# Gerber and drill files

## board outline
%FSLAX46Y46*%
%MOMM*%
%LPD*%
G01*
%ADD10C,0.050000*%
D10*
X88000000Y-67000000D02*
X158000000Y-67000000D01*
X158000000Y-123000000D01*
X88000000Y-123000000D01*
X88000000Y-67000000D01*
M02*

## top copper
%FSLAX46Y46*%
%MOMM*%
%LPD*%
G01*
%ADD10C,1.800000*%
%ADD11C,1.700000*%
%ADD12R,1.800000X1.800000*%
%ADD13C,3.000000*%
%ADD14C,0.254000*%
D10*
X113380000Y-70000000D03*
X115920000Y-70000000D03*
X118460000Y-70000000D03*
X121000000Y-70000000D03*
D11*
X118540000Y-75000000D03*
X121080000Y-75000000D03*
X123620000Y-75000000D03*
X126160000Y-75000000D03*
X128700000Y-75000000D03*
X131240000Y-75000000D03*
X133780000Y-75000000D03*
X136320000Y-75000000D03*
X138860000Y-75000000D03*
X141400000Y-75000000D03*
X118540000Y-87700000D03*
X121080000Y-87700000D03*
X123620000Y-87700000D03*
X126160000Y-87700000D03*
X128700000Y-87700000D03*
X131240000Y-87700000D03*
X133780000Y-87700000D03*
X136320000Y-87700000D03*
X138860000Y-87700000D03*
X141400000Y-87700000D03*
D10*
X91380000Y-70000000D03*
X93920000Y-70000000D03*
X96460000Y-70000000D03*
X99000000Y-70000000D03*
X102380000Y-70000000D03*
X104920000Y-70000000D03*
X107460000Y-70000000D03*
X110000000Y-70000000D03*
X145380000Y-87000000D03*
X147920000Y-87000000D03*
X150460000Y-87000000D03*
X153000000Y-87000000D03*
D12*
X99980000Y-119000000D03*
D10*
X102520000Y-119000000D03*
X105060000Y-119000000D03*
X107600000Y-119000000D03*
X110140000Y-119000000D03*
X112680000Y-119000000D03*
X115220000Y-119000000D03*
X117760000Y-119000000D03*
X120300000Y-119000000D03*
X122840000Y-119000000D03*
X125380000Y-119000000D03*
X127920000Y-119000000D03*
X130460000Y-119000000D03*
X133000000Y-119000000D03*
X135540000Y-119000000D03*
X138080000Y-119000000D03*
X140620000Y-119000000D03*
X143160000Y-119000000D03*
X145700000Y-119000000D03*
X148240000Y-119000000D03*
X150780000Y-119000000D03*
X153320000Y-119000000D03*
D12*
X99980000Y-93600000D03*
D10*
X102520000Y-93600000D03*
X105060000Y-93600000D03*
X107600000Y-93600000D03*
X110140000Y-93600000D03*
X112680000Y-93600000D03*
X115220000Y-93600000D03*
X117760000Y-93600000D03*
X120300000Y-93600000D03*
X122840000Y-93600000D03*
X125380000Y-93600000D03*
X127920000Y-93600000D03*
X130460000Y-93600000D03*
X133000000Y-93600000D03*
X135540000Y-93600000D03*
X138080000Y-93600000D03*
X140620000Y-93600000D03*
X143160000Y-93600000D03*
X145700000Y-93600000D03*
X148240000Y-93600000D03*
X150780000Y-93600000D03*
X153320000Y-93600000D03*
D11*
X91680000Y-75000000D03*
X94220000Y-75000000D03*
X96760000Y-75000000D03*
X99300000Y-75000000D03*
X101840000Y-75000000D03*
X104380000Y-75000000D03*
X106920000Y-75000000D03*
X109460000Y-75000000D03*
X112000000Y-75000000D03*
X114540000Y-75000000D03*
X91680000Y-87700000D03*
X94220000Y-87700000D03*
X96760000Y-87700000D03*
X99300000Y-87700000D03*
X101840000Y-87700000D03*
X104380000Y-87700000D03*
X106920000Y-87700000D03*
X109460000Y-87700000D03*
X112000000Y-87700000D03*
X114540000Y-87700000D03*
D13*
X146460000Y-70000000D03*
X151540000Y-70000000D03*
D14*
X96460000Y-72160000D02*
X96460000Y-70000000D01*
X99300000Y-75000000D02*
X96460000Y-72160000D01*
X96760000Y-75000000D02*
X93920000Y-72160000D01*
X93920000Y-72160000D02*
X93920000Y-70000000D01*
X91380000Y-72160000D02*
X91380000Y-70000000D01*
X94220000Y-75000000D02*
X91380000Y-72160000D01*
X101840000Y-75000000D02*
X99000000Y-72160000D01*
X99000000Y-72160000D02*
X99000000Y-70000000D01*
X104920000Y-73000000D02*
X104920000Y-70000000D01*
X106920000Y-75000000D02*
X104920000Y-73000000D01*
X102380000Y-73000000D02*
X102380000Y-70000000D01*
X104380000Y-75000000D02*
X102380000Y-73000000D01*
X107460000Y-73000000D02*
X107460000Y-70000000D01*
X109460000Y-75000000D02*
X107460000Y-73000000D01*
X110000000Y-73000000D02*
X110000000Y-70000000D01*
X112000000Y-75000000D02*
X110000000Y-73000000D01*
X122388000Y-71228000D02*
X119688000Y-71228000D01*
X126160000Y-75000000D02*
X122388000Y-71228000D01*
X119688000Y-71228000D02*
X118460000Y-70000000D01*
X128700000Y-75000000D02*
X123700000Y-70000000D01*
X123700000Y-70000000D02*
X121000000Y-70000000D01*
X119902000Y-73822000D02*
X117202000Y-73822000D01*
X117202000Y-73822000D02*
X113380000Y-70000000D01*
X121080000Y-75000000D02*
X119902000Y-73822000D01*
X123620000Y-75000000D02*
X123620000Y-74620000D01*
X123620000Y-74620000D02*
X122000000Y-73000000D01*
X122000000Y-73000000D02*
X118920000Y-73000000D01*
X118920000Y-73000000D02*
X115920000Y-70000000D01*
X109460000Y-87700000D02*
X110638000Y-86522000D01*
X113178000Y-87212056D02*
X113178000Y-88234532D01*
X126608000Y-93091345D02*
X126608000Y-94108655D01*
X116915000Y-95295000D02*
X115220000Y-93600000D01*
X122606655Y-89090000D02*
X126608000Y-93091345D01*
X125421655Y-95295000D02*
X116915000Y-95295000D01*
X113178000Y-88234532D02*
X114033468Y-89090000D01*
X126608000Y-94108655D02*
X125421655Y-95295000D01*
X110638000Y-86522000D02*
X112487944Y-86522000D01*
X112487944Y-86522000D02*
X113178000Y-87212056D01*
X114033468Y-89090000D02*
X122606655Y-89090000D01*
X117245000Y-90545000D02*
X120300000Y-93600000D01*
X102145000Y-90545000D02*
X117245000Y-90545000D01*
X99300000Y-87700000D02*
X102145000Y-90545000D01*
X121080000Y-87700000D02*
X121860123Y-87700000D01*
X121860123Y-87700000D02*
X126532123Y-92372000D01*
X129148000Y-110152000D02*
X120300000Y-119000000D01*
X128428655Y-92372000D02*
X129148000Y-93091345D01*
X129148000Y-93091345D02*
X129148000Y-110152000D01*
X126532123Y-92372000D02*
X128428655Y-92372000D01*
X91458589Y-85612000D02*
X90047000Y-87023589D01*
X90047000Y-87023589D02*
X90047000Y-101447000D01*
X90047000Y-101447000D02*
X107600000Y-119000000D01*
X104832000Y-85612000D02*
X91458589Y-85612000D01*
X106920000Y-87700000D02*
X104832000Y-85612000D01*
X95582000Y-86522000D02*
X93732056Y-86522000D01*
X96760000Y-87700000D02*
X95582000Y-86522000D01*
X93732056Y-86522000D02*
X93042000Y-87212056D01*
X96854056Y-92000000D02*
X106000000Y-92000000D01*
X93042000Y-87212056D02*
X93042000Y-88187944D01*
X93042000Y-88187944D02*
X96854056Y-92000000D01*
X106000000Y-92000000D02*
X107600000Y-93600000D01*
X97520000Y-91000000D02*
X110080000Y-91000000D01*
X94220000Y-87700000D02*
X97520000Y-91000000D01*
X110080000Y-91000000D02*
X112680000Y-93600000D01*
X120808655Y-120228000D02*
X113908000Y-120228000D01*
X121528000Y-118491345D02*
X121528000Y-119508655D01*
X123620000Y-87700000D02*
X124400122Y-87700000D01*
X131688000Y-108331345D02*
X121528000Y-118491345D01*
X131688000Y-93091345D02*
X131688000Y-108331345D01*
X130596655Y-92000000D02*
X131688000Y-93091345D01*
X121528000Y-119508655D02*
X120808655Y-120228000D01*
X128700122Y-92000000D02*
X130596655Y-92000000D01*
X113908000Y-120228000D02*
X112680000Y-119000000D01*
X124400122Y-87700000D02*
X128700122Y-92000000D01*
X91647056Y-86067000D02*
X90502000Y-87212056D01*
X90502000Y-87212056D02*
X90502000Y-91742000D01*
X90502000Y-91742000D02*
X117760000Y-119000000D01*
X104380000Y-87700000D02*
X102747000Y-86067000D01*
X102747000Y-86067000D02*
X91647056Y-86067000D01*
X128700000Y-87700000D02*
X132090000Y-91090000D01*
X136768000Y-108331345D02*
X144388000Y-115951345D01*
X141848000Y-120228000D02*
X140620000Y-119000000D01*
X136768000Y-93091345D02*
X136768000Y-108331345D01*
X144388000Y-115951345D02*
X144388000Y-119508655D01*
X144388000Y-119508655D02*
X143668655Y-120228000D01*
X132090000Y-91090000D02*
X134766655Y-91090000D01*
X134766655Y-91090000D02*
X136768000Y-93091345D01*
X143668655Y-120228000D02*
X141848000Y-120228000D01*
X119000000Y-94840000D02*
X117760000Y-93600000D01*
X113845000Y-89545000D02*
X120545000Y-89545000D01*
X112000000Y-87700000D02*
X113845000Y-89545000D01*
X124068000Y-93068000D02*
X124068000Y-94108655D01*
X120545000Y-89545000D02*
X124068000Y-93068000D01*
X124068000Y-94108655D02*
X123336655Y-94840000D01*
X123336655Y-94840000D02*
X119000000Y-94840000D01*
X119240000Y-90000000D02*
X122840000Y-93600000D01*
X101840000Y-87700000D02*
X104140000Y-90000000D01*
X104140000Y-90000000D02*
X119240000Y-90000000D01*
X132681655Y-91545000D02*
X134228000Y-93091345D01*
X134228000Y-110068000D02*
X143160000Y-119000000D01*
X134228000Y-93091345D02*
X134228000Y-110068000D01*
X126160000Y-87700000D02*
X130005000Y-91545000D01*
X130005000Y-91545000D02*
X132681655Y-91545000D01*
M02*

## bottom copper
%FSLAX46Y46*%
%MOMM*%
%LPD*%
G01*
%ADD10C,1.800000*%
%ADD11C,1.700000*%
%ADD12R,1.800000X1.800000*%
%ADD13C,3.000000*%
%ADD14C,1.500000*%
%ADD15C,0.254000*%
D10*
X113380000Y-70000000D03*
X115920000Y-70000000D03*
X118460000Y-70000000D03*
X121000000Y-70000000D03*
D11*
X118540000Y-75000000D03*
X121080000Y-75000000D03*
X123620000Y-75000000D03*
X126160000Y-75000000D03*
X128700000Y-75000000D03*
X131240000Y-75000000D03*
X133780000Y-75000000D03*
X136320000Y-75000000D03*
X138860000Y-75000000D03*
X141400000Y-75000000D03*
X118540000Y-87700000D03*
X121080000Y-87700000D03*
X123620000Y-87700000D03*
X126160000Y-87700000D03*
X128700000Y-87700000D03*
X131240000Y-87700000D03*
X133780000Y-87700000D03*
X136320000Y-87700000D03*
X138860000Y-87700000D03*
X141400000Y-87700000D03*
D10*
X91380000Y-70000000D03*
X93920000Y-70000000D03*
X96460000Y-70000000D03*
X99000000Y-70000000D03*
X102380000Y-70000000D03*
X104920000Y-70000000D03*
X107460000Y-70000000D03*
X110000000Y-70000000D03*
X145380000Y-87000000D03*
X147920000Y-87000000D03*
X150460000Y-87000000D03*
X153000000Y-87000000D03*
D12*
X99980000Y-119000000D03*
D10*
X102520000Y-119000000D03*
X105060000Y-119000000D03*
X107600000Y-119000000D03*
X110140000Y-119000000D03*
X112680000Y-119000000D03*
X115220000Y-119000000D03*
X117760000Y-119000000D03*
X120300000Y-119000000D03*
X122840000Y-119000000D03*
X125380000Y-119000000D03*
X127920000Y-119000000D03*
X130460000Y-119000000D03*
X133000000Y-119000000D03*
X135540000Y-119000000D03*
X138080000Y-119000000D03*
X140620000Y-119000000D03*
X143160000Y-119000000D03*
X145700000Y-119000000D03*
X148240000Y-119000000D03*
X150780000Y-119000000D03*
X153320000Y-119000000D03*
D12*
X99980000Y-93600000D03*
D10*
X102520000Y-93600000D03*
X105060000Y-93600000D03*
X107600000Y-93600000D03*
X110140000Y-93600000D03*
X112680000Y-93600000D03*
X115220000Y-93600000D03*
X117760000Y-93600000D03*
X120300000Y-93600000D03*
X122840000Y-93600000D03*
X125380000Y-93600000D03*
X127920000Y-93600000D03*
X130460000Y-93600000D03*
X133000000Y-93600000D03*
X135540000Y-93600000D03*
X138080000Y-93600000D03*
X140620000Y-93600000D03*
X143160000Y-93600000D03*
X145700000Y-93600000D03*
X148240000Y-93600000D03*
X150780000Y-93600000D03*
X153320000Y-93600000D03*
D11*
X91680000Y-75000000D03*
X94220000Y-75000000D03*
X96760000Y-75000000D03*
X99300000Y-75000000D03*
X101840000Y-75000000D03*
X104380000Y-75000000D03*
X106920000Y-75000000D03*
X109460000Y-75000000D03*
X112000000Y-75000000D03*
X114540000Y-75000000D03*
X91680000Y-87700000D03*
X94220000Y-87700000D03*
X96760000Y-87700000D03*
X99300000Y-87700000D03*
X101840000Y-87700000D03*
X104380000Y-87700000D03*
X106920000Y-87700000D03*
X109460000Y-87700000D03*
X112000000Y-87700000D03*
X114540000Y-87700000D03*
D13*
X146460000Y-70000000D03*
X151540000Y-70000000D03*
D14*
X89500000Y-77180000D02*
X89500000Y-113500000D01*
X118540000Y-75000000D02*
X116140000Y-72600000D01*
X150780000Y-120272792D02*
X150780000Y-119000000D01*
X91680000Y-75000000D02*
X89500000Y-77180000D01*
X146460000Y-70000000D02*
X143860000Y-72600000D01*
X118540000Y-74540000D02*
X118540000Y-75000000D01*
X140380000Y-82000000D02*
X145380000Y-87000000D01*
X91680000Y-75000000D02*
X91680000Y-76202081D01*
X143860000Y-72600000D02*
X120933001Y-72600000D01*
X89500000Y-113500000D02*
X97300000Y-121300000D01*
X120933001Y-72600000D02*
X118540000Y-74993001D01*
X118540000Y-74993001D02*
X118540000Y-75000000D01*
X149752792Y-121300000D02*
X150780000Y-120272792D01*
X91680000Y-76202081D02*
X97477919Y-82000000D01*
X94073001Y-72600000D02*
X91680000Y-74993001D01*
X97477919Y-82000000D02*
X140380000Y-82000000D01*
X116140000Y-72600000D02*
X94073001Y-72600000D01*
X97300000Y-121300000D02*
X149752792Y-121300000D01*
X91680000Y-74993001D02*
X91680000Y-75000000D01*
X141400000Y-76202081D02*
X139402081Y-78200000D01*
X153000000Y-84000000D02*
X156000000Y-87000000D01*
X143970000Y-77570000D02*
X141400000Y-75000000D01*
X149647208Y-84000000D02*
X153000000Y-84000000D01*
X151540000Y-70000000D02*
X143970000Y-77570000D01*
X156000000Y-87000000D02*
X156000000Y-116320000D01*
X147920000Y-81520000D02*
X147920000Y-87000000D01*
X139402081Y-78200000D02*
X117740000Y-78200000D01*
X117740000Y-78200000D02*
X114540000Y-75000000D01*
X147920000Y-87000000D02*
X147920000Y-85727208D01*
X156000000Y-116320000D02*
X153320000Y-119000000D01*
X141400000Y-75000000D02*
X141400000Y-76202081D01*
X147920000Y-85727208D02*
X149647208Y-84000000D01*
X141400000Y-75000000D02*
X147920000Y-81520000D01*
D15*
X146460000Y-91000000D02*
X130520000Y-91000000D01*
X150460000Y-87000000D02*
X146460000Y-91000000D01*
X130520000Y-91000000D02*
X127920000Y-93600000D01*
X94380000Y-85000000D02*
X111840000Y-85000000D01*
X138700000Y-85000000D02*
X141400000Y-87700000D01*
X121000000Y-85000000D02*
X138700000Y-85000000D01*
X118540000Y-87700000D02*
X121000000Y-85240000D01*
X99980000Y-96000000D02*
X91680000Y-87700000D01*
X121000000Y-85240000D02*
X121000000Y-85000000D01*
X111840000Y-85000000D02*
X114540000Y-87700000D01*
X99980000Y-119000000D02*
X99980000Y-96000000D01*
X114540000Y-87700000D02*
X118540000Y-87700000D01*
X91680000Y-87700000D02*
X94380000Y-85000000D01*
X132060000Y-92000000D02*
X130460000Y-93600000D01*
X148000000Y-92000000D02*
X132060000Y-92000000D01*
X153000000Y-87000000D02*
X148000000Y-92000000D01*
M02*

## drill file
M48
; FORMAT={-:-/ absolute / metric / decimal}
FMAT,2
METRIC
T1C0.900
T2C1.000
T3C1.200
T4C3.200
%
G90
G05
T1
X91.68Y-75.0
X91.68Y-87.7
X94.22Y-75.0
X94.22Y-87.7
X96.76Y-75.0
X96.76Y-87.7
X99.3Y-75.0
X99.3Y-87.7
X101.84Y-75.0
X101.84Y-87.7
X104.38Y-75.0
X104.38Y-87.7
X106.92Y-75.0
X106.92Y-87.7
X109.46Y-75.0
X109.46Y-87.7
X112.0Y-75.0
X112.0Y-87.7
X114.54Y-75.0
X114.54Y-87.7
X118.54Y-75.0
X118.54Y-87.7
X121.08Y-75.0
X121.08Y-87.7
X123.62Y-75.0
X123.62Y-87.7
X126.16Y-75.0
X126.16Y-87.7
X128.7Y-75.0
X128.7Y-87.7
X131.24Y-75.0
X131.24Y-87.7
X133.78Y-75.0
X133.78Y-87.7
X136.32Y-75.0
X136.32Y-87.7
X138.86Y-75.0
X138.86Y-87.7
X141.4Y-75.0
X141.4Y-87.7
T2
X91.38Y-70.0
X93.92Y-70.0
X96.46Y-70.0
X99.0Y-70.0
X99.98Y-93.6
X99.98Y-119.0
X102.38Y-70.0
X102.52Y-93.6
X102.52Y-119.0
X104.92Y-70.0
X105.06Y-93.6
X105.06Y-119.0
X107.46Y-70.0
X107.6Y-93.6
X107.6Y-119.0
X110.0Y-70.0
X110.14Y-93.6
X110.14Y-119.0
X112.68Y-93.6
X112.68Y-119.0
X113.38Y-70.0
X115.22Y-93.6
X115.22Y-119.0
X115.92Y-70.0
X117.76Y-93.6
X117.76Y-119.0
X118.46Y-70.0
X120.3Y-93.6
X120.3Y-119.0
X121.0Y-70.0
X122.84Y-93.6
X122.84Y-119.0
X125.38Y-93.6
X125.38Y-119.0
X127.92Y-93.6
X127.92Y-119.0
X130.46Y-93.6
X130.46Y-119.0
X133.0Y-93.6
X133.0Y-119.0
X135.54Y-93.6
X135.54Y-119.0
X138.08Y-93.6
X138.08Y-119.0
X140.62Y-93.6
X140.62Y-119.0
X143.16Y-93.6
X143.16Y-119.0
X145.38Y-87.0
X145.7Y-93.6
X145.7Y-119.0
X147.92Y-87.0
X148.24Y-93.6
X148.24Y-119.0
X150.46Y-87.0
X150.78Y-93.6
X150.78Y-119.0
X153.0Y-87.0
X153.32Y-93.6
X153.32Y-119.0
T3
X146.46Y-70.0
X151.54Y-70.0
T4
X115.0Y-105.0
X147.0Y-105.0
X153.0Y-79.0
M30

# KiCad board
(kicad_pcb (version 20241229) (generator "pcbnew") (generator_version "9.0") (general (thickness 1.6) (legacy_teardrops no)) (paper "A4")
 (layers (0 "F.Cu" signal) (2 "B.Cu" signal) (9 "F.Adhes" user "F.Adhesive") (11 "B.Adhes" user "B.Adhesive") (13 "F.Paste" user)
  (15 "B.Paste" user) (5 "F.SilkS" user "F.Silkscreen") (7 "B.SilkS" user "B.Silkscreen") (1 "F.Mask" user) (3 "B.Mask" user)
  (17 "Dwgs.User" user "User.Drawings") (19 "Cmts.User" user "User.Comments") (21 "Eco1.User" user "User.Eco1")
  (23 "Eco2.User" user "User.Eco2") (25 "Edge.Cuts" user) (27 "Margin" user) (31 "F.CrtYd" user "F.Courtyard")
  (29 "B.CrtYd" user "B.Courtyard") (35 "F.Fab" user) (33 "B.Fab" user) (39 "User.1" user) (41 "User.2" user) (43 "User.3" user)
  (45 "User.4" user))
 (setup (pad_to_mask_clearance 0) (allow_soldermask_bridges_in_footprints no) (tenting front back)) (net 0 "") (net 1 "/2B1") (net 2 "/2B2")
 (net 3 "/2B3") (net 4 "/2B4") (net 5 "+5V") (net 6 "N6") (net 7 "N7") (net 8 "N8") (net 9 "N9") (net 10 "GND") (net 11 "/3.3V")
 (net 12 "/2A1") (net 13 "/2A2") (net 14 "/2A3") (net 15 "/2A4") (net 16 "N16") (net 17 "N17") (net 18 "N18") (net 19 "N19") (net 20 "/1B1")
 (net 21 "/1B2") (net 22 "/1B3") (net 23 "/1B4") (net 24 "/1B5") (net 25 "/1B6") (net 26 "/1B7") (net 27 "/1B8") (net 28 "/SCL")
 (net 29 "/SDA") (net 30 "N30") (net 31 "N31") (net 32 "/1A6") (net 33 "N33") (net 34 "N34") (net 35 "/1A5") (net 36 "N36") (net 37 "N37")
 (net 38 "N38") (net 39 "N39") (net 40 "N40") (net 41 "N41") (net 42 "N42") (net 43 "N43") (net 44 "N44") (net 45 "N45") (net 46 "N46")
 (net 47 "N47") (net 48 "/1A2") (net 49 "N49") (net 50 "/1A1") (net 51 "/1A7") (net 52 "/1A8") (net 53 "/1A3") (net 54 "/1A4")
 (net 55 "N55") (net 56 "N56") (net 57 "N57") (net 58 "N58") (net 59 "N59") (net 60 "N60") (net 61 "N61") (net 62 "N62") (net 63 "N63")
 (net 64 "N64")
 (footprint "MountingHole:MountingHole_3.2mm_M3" (layer "F.Cu") (at 153 79)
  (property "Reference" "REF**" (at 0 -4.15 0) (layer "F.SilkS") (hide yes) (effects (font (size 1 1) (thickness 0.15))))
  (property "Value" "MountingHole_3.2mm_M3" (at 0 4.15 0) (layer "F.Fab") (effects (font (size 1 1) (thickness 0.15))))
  (pad "" np_thru_hole circle (at 0 0) (size 3.2 3.2) (drill 3.2) (layers "*.Cu" "*.Mask")))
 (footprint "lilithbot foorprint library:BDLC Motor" (layer "F.Cu") (at 117.19 70.254)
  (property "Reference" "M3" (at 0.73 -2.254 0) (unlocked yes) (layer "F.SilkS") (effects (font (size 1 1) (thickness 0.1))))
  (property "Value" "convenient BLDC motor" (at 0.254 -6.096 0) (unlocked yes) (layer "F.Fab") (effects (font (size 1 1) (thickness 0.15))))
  (pad "1" thru_hole circle (at -3.81 -0.254) (size 1.8 1.8) (drill 1) (layers "*.Cu" "*.Mask") (remove_unused_layers no) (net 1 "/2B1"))
  (pad "2" thru_hole circle (at -1.27 -0.254) (size 1.8 1.8) (drill 1) (layers "*.Cu" "*.Mask") (remove_unused_layers no) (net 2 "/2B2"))
  (pad "3" thru_hole circle (at 1.27 -0.254) (size 1.8 1.8) (drill 1) (layers "*.Cu" "*.Mask") (remove_unused_layers no) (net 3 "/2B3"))
  (pad "4" thru_hole circle (at 3.81 -0.254) (size 1.8 1.8) (drill 1) (layers "*.Cu" "*.Mask") (remove_unused_layers no) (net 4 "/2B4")))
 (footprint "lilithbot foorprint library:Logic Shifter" (layer "F.Cu") (at 130.944878 82.58)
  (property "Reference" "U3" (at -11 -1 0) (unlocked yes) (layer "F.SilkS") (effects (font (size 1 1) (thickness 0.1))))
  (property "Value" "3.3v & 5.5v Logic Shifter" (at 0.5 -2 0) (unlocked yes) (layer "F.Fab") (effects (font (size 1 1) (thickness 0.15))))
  (pad "1" thru_hole circle (at -12.404878 -7.58) (size 1.7 1.7) (drill 0.9) (layers "*.Cu" "*.Mask") (remove_unused_layers no)
   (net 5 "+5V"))
  (pad "2" thru_hole circle (at -9.864878 -7.58) (size 1.7 1.7) (drill 0.9) (layers "*.Cu" "*.Mask") (remove_unused_layers no)
   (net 1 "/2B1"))
  (pad "3" thru_hole circle (at -7.324878 -7.58) (size 1.7 1.7) (drill 0.9) (layers "*.Cu" "*.Mask") (remove_unused_layers no)
   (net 2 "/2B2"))
  (pad "4" thru_hole circle (at -4.784878 -7.58) (size 1.7 1.7) (drill 0.9) (layers "*.Cu" "*.Mask") (remove_unused_layers no)
   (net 3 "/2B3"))
  (pad "5" thru_hole circle (at -2.244878 -7.58) (size 1.7 1.7) (drill 0.9) (layers "*.Cu" "*.Mask") (remove_unused_layers no)
   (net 4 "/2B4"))
  (pad "6" thru_hole circle (at 0.295122 -7.58) (size 1.7 1.7) (drill 0.9) (layers "*.Cu" "*.Mask") (remove_unused_layers no) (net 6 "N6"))
  (pad "7" thru_hole circle (at 2.835122 -7.58) (size 1.7 1.7) (drill 0.9) (layers "*.Cu" "*.Mask") (remove_unused_layers no) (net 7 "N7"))
  (pad "8" thru_hole circle (at 5.375122 -7.58) (size 1.7 1.7) (drill 0.9) (layers "*.Cu" "*.Mask") (remove_unused_layers no) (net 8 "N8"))
  (pad "9" thru_hole circle (at 7.915122 -7.58) (size 1.7 1.7) (drill 0.9) (layers "*.Cu" "*.Mask") (remove_unused_layers no) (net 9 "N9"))
  (pad "10" thru_hole circle (at 10.455122 -7.58) (size 1.7 1.7) (drill 0.9) (layers "*.Cu" "*.Mask") (remove_unused_layers no)
   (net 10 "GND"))
  (pad "11" thru_hole circle (at -12.404878 5.12) (size 1.7 1.7) (drill 0.9) (layers "*.Cu" "*.Mask") (remove_unused_layers no)
   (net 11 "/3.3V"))
  (pad "12" thru_hole circle (at -9.864878 5.12) (size 1.7 1.7) (drill 0.9) (layers "*.Cu" "*.Mask") (remove_unused_layers no)
   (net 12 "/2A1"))
  (pad "13" thru_hole circle (at -7.324878 5.12) (size 1.7 1.7) (drill 0.9) (layers "*.Cu" "*.Mask") (remove_unused_layers no)
   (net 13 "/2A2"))
  (pad "14" thru_hole circle (at -4.784878 5.12) (size 1.7 1.7) (drill 0.9) (layers "*.Cu" "*.Mask") (remove_unused_layers no)
   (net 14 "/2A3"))
  (pad "15" thru_hole circle (at -2.244878 5.12) (size 1.7 1.7) (drill 0.9) (layers "*.Cu" "*.Mask") (remove_unused_layers no)
   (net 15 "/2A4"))
  (pad "16" thru_hole circle (at 0.295122 5.12) (size 1.7 1.7) (drill 0.9) (layers "*.Cu" "*.Mask") (remove_unused_layers no) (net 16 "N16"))
  (pad "17" thru_hole circle (at 2.835122 5.12) (size 1.7 1.7) (drill 0.9) (layers "*.Cu" "*.Mask") (remove_unused_layers no) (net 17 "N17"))
  (pad "18" thru_hole circle (at 5.375122 5.12) (size 1.7 1.7) (drill 0.9) (layers "*.Cu" "*.Mask") (remove_unused_layers no) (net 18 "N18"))
  (pad "19" thru_hole circle (at 7.915122 5.12) (size 1.7 1.7) (drill 0.9) (layers "*.Cu" "*.Mask") (remove_unused_layers no) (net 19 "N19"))
  (pad "20" thru_hole circle (at 10.455122 5.12) (size 1.7 1.7) (drill 0.9) (layers "*.Cu" "*.Mask") (remove_unused_layers no)
   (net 11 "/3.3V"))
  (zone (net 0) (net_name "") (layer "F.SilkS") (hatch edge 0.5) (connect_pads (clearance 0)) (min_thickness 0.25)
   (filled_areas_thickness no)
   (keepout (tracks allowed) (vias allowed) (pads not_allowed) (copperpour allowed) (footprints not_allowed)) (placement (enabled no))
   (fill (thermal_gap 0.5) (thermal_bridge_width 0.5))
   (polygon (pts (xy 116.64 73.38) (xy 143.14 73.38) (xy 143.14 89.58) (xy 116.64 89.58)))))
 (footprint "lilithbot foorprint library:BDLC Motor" (layer "F.Cu") (at 95.19 70.254)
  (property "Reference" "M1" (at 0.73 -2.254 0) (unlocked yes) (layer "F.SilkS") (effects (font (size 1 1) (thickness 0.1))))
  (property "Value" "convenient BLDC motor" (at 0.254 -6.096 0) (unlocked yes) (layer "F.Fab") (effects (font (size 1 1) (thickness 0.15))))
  (pad "1" thru_hole circle (at -3.81 -0.254) (size 1.8 1.8) (drill 1) (layers "*.Cu" "*.Mask") (remove_unused_layers no) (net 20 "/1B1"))
  (pad "2" thru_hole circle (at -1.27 -0.254) (size 1.8 1.8) (drill 1) (layers "*.Cu" "*.Mask") (remove_unused_layers no) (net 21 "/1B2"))
  (pad "3" thru_hole circle (at 1.27 -0.254) (size 1.8 1.8) (drill 1) (layers "*.Cu" "*.Mask") (remove_unused_layers no) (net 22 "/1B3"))
  (pad "4" thru_hole circle (at 3.81 -0.254) (size 1.8 1.8) (drill 1) (layers "*.Cu" "*.Mask") (remove_unused_layers no) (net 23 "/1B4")))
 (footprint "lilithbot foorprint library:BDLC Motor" (layer "F.Cu") (at 106.19 70.254)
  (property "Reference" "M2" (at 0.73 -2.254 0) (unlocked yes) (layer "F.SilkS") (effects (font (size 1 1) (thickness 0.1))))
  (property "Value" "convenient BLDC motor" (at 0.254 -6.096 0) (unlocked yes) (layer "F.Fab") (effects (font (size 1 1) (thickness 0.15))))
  (pad "1" thru_hole circle (at -3.81 -0.254) (size 1.8 1.8) (drill 1) (layers "*.Cu" "*.Mask") (remove_unused_layers no) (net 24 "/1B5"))
  (pad "2" thru_hole circle (at -1.27 -0.254) (size 1.8 1.8) (drill 1) (layers "*.Cu" "*.Mask") (remove_unused_layers no) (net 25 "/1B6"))
  (pad "3" thru_hole circle (at 1.27 -0.254) (size 1.8 1.8) (drill 1) (layers "*.Cu" "*.Mask") (remove_unused_layers no) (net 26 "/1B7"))
  (pad "4" thru_hole circle (at 3.81 -0.254) (size 1.8 1.8) (drill 1) (layers "*.Cu" "*.Mask") (remove_unused_layers no) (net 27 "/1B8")))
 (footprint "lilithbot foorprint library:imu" (layer "F.Cu") (at 149.19 87)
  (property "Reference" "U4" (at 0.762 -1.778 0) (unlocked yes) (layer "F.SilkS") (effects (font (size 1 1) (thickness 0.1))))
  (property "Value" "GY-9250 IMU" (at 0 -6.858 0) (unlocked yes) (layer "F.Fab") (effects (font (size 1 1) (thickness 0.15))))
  (pad "1" thru_hole circle (at -3.81 0) (size 1.8 1.8) (drill 1) (layers "*.Cu" "*.Mask") (remove_unused_layers no) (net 5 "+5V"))
  (pad "2" thru_hole circle (at -1.27 0) (size 1.8 1.8) (drill 1) (layers "*.Cu" "*.Mask") (remove_unused_layers no) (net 10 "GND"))
  (pad "3" thru_hole circle (at 1.27 0) (size 1.8 1.8) (drill 1) (layers "*.Cu" "*.Mask") (remove_unused_layers no) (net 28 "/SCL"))
  (pad "4" thru_hole circle (at 3.81 0) (size 1.8 1.8) (drill 1) (layers "*.Cu" "*.Mask") (remove_unused_layers no) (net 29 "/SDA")))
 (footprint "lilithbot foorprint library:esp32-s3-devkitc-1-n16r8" (layer "F.Cu") (at 125.38 106.3 90)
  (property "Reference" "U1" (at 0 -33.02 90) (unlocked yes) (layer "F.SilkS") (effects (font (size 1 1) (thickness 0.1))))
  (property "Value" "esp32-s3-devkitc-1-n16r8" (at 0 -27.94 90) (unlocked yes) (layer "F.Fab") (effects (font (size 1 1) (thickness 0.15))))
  (pad "1" thru_hole rect (at -12.7 -25.4 90) (size 1.8 1.8) (drill 1) (layers "*.Cu" "*.Mask") (remove_unused_layers no) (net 11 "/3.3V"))
  (pad "2" thru_hole circle (at -12.7 -22.86 90) (size 1.8 1.8) (drill 1) (layers "*.Cu" "*.Mask") (remove_unused_layers no) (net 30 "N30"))
  (pad "3" thru_hole circle (at -12.7 -20.32 90) (size 1.8 1.8) (drill 1) (layers "*.Cu" "*.Mask") (remove_unused_layers no) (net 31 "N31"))
  (pad "4" thru_hole circle (at -12.7 -17.78 90) (size 1.8 1.8) (drill 1) (layers "*.Cu" "*.Mask") (remove_unused_layers no) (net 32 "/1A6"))
  (pad "5" thru_hole circle (at -12.7 -15.24 90) (size 1.8 1.8) (drill 1) (layers "*.Cu" "*.Mask") (remove_unused_layers no) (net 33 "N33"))
  (pad "6" thru_hole circle (at -12.7 -12.7 90) (size 1.8 1.8) (drill 1) (layers "*.Cu" "*.Mask") (remove_unused_layers no) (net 13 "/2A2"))
  (pad "7" thru_hole circle (at -12.7 -10.16 90) (size 1.8 1.8) (drill 1) (layers "*.Cu" "*.Mask") (remove_unused_layers no) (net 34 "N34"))
  (pad "8" thru_hole circle (at -12.7 -7.62 90) (size 1.8 1.8) (drill 1) (layers "*.Cu" "*.Mask") (remove_unused_layers no) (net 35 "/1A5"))
  (pad "9" thru_hole circle (at -12.7 -5.08 90) (size 1.8 1.8) (drill 1) (layers "*.Cu" "*.Mask") (remove_unused_layers no) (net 12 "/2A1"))
  (pad "10" thru_hole circle (at -12.7 -2.54 90) (size 1.8 1.8) (drill 1) (layers "*.Cu" "*.Mask") (remove_unused_layers no) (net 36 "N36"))
  (pad "11" thru_hole circle (at -12.7 0 90) (size 1.8 1.8) (drill 1) (layers "*.Cu" "*.Mask") (remove_unused_layers no) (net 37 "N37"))
  (pad "12" thru_hole circle (at -12.7 2.54 90) (size 1.8 1.8) (drill 1) (layers "*.Cu" "*.Mask") (remove_unused_layers no) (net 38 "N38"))
  (pad "13" thru_hole circle (at -12.7 5.08 90) (size 1.8 1.8) (drill 1) (layers "*.Cu" "*.Mask") (remove_unused_layers no) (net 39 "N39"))
  (pad "14" thru_hole circle (at -12.7 7.62 90) (size 1.8 1.8) (drill 1) (layers "*.Cu" "*.Mask") (remove_unused_layers no) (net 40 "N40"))
  (pad "15" thru_hole circle (at -12.7 10.16 90) (size 1.8 1.8) (drill 1) (layers "*.Cu" "*.Mask") (remove_unused_layers no) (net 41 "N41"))
  (pad "16" thru_hole circle (at -12.7 12.7 90) (size 1.8 1.8) (drill 1) (layers "*.Cu" "*.Mask") (remove_unused_layers no) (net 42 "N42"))
  (pad "17" thru_hole circle (at -12.7 15.24 90) (size 1.8 1.8) (drill 1) (layers "*.Cu" "*.Mask") (remove_unused_layers no) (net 15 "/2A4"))
  (pad "18" thru_hole circle (at -12.7 17.78 90) (size 1.8 1.8) (drill 1) (layers "*.Cu" "*.Mask") (remove_unused_layers no) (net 14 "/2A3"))
  (pad "19" thru_hole circle (at -12.7 20.32 90) (size 1.8 1.8) (drill 1) (layers "*.Cu" "*.Mask") (remove_unused_layers no) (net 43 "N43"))
  (pad "20" thru_hole circle (at -12.7 22.86 90) (size 1.8 1.8) (drill 1) (layers "*.Cu" "*.Mask") (remove_unused_layers no) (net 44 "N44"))
  (pad "21" thru_hole circle (at -12.7 25.4 90) (size 1.8 1.8) (drill 1) (layers "*.Cu" "*.Mask") (remove_unused_layers no) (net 5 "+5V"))
  (pad "22" thru_hole circle (at -12.7 27.94 90) (size 1.8 1.8) (drill 1) (layers "*.Cu" "*.Mask") (remove_unused_layers no) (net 10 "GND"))
  (pad "23" thru_hole rect (at 12.7 -25.4 90) (size 1.8 1.8) (drill 1) (layers "*.Cu" "*.Mask") (remove_unused_layers no) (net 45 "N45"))
  (pad "24" thru_hole circle (at 12.7 -22.86 90) (size 1.8 1.8) (drill 1) (layers "*.Cu" "*.Mask") (remove_unused_layers no) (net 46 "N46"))
  (pad "25" thru_hole circle (at 12.7 -20.32 90) (size 1.8 1.8) (drill 1) (layers "*.Cu" "*.Mask") (remove_unused_layers no) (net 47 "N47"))
  (pad "26" thru_hole circle (at 12.7 -17.78 90) (size 1.8 1.8) (drill 1) (layers "*.Cu" "*.Mask") (remove_unused_layers no) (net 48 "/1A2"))
  (pad "27" thru_hole circle (at 12.7 -15.24 90) (size 1.8 1.8) (drill 1) (layers "*.Cu" "*.Mask") (remove_unused_layers no) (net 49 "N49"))
  (pad "28" thru_hole circle (at 12.7 -12.7 90) (size 1.8 1.8) (drill 1) (layers "*.Cu" "*.Mask") (remove_unused_layers no) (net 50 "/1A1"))
  (pad "29" thru_hole circle (at 12.7 -10.16 90) (size 1.8 1.8) (drill 1) (layers "*.Cu" "*.Mask") (remove_unused_layers no) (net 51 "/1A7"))
  (pad "30" thru_hole circle (at 12.7 -7.62 90) (size 1.8 1.8) (drill 1) (layers "*.Cu" "*.Mask") (remove_unused_layers no) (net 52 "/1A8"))
  (pad "31" thru_hole circle (at 12.7 -5.08 90) (size 1.8 1.8) (drill 1) (layers "*.Cu" "*.Mask") (remove_unused_layers no) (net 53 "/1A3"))
  (pad "32" thru_hole circle (at 12.7 -2.54 90) (size 1.8 1.8) (drill 1) (layers "*.Cu" "*.Mask") (remove_unused_layers no) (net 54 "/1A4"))
  (pad "33" thru_hole circle (at 12.7 0 90) (size 1.8 1.8) (drill 1) (layers "*.Cu" "*.Mask") (remove_unused_layers no) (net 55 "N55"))
  (pad "34" thru_hole circle (at 12.7 2.54 90) (size 1.8 1.8) (drill 1) (layers "*.Cu" "*.Mask") (remove_unused_layers no) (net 28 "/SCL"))
  (pad "35" thru_hole circle (at 12.7 5.08 90) (size 1.8 1.8) (drill 1) (layers "*.Cu" "*.Mask") (remove_unused_layers no) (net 29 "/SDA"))
  (pad "36" thru_hole circle (at 12.7 7.62 90) (size 1.8 1.8) (drill 1) (layers "*.Cu" "*.Mask") (remove_unused_layers no) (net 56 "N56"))
  (pad "37" thru_hole circle (at 12.7 10.16 90) (size 1.8 1.8) (drill 1) (layers "*.Cu" "*.Mask") (remove_unused_layers no) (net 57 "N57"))
  (pad "38" thru_hole circle (at 12.7 12.7 90) (size 1.8 1.8) (drill 1) (layers "*.Cu" "*.Mask") (remove_unused_layers no) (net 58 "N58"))
  (pad "39" thru_hole circle (at 12.7 15.24 90) (size 1.8 1.8) (drill 1) (layers "*.Cu" "*.Mask") (remove_unused_layers no) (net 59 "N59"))
  (pad "40" thru_hole circle (at 12.7 17.78 90) (size 1.8 1.8) (drill 1) (layers "*.Cu" "*.Mask") (remove_unused_layers no) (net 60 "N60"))
  (pad "41" thru_hole circle (at 12.7 20.32 90) (size 1.8 1.8) (drill 1) (layers "*.Cu" "*.Mask") (remove_unused_layers no) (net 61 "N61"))
  (pad "42" thru_hole circle (at 12.7 22.86 90) (size 1.8 1.8) (drill 1) (layers "*.Cu" "*.Mask") (remove_unused_layers no) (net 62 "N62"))
  (pad "43" thru_hole circle (at 12.7 25.4 90) (size 1.8 1.8) (drill 1) (layers "*.Cu" "*.Mask") (remove_unused_layers no) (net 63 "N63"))
  (pad "44" thru_hole circle (at 12.7 27.94 90) (size 1.8 1.8) (drill 1) (layers "*.Cu" "*.Mask") (remove_unused_layers no) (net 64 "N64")))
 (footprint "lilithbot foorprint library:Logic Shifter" (layer "F.Cu") (at 104.084878 82.58)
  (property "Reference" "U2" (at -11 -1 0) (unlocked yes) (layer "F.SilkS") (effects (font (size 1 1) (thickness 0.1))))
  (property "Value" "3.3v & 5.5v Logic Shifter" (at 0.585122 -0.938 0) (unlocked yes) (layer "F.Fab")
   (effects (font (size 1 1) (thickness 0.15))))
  (pad "1" thru_hole circle (at -12.404878 -7.58) (size 1.7 1.7) (drill 0.9) (layers "*.Cu" "*.Mask") (remove_unused_layers no)
   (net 5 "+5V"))
  (pad "2" thru_hole circle (at -9.864878 -7.58) (size 1.7 1.7) (drill 0.9) (layers "*.Cu" "*.Mask") (remove_unused_layers no)
   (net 20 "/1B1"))
  (pad "3" thru_hole circle (at -7.324878 -7.58) (size 1.7 1.7) (drill 0.9) (layers "*.Cu" "*.Mask") (remove_unused_layers no)
   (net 21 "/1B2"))
  (pad "4" thru_hole circle (at -4.784878 -7.58) (size 1.7 1.7) (drill 0.9) (layers "*.Cu" "*.Mask") (remove_unused_layers no)
   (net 22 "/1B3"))
  (pad "5" thru_hole circle (at -2.244878 -7.58) (size 1.7 1.7) (drill 0.9) (layers "*.Cu" "*.Mask") (remove_unused_layers no)
   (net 23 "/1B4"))
  (pad "6" thru_hole circle (at 0.295122 -7.58) (size 1.7 1.7) (drill 0.9) (layers "*.Cu" "*.Mask") (remove_unused_layers no)
   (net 24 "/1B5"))
  (pad "7" thru_hole circle (at 2.835122 -7.58) (size 1.7 1.7) (drill 0.9) (layers "*.Cu" "*.Mask") (remove_unused_layers no)
   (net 25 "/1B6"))
  (pad "8" thru_hole circle (at 5.375122 -7.58) (size 1.7 1.7) (drill 0.9) (layers "*.Cu" "*.Mask") (remove_unused_layers no)
   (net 26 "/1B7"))
  (pad "9" thru_hole circle (at 7.915122 -7.58) (size 1.7 1.7) (drill 0.9) (layers "*.Cu" "*.Mask") (remove_unused_layers no)
   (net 27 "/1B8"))
  (pad "10" thru_hole circle (at 10.455122 -7.58) (size 1.7 1.7) (drill 0.9) (layers "*.Cu" "*.Mask") (remove_unused_layers no)
   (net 10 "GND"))
  (pad "11" thru_hole circle (at -12.404878 5.12) (size 1.7 1.7) (drill 0.9) (layers "*.Cu" "*.Mask") (remove_unused_layers no)
   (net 11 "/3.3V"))
  (pad "12" thru_hole circle (at -9.864878 5.12) (size 1.7 1.7) (drill 0.9) (layers "*.Cu" "*.Mask") (remove_unused_layers no)
   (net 50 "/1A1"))
  (pad "13" thru_hole circle (at -7.324878 5.12) (size 1.7 1.7) (drill 0.9) (layers "*.Cu" "*.Mask") (remove_unused_layers no)
   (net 48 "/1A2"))
  (pad "14" thru_hole circle (at -4.784878 5.12) (size 1.7 1.7) (drill 0.9) (layers "*.Cu" "*.Mask") (remove_unused_layers no)
   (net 53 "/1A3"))
  (pad "15" thru_hole circle (at -2.244878 5.12) (size 1.7 1.7) (drill 0.9) (layers "*.Cu" "*.Mask") (remove_unused_layers no)
   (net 54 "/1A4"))
  (pad "16" thru_hole circle (at 0.295122 5.12) (size 1.7 1.7) (drill 0.9) (layers "*.Cu" "*.Mask") (remove_unused_layers no)
   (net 35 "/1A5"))
  (pad "17" thru_hole circle (at 2.835122 5.12) (size 1.7 1.7) (drill 0.9) (layers "*.Cu" "*.Mask") (remove_unused_layers no)
   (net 32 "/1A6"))
  (pad "18" thru_hole circle (at 5.375122 5.12) (size 1.7 1.7) (drill 0.9) (layers "*.Cu" "*.Mask") (remove_unused_layers no)
   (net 51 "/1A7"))
  (pad "19" thru_hole circle (at 7.915122 5.12) (size 1.7 1.7) (drill 0.9) (layers "*.Cu" "*.Mask") (remove_unused_layers no)
   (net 52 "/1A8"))
  (pad "20" thru_hole circle (at 10.455122 5.12) (size 1.7 1.7) (drill 0.9) (layers "*.Cu" "*.Mask") (remove_unused_layers no)
   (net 11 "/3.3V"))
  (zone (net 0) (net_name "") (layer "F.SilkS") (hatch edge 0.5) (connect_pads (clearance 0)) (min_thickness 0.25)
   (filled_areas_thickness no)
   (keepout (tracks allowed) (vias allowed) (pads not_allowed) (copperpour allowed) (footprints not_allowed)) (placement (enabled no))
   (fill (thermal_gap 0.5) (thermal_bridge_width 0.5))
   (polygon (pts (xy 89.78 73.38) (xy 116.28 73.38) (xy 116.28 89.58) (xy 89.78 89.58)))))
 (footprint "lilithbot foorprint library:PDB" (layer "F.Cu") (at 149 70)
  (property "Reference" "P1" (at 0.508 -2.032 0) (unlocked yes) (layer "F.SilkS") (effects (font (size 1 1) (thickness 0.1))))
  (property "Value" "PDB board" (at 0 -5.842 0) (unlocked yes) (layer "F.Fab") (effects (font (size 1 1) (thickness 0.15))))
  (pad "1" thru_hole circle (at -2.54 0) (size 3 3) (drill 1.2) (layers "*.Cu" "*.Mask") (remove_unused_layers no) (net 5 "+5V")
   (thermal_bridge_width 0.5) (thermal_bridge_angle 90) (thermal_gap 0.25))
  (pad "2" thru_hole circle (at 2.54 0) (size 3 3) (drill 1.2) (layers "*.Cu" "*.Mask") (remove_unused_layers no) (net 10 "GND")
   (thermal_bridge_width 0.5) (thermal_bridge_angle 90) (thermal_gap 0.25)))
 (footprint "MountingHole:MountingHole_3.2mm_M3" (layer "F.Cu") (at 147 105)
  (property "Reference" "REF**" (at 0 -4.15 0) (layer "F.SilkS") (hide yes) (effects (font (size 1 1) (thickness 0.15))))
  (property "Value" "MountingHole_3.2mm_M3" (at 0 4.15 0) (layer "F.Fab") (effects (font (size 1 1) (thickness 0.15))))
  (pad "" np_thru_hole circle (at 0 0) (size 3.2 3.2) (drill 3.2) (layers "*.Cu" "*.Mask")))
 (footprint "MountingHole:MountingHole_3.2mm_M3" (layer "F.Cu") (at 115 105)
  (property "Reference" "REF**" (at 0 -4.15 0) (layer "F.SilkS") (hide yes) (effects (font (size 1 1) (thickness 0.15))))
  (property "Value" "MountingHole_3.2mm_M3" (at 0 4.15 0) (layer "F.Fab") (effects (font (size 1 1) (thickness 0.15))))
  (pad "" np_thru_hole circle (at 0 0) (size 3.2 3.2) (drill 3.2) (layers "*.Cu" "*.Mask")))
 (gr_rect (start 88 67) (end 158 123) (stroke (width 0.05) (type solid)) (fill no) (layer "Edge.Cuts"))
 (segment (start 96.46 72.16) (end 96.46 70) (width 0.254) (layer "F.Cu") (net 22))
 (segment (start 99.3 75) (end 96.46 72.16) (width 0.254) (layer "F.Cu") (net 22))
 (segment (start 96.76 75) (end 93.92 72.16) (width 0.254) (layer "F.Cu") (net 21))
 (segment (start 93.92 72.16) (end 93.92 70) (width 0.254) (layer "F.Cu") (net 21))
 (segment (start 91.38 72.16) (end 91.38 70) (width 0.254) (layer "F.Cu") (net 20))
 (segment (start 94.22 75) (end 91.38 72.16) (width 0.254) (layer "F.Cu") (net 20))
 (segment (start 101.84 75) (end 99 72.16) (width 0.254) (layer "F.Cu") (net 23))
 (segment (start 99 72.16) (end 99 70) (width 0.254) (layer "F.Cu") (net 23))
 (segment (start 104.92 73) (end 104.92 70) (width 0.254) (layer "F.Cu") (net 25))
 (segment (start 106.92 75) (end 104.92 73) (width 0.254) (layer "F.Cu") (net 25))
 (segment (start 102.38 73) (end 102.38 70) (width 0.254) (layer "F.Cu") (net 24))
 (segment (start 104.38 75) (end 102.38 73) (width 0.254) (layer "F.Cu") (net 24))
 (segment (start 107.46 73) (end 107.46 70) (width 0.254) (layer "F.Cu") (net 26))
 (segment (start 109.46 75) (end 107.46 73) (width 0.254) (layer "F.Cu") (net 26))
 (segment (start 110 73) (end 110 70) (width 0.254) (layer "F.Cu") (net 27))
 (segment (start 112 75) (end 110 73) (width 0.254) (layer "F.Cu") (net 27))
 (segment (start 122.388 71.228) (end 119.688 71.228) (width 0.254) (layer "F.Cu") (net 3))
 (segment (start 126.16 75) (end 122.388 71.228) (width 0.254) (layer "F.Cu") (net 3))
 (segment (start 119.688 71.228) (end 118.46 70) (width 0.254) (layer "F.Cu") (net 3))
 (segment (start 128.7 75) (end 123.7 70) (width 0.254) (layer "F.Cu") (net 4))
 (segment (start 123.7 70) (end 121 70) (width 0.254) (layer "F.Cu") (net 4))
 (segment (start 119.902 73.822) (end 117.202 73.822) (width 0.254) (layer "F.Cu") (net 1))
 (segment (start 117.202 73.822) (end 113.38 70) (width 0.254) (layer "F.Cu") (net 1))
 (segment (start 121.08 75) (end 119.902 73.822) (width 0.254) (layer "F.Cu") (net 1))
 (segment (start 123.62 75) (end 123.62 74.62) (width 0.254) (layer "F.Cu") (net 2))
 (segment (start 123.62 74.62) (end 122 73) (width 0.254) (layer "F.Cu") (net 2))
 (segment (start 122 73) (end 118.92 73) (width 0.254) (layer "F.Cu") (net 2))
 (segment (start 118.92 73) (end 115.92 70) (width 0.254) (layer "F.Cu") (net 2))
 (segment (start 89.5 77.18) (end 89.5 113.5) (width 1.5) (layer "B.Cu") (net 5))
 (segment (start 118.54 75) (end 116.14 72.6) (width 1.5) (layer "B.Cu") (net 5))
 (segment (start 150.78 120.272792) (end 150.78 119) (width 1.5) (layer "B.Cu") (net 5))
 (segment (start 91.68 75) (end 89.5 77.18) (width 1.5) (layer "B.Cu") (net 5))
 (segment (start 146.46 70) (end 143.86 72.6) (width 1.5) (layer "B.Cu") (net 5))
 (segment (start 118.54 74.54) (end 118.54 75) (width 1.5) (layer "B.Cu") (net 5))
 (segment (start 140.38 82) (end 145.38 87) (width 1.5) (layer "B.Cu") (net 5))
 (segment (start 91.68 75) (end 91.68 76.202081) (width 1.5) (layer "B.Cu") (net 5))
 (segment (start 143.86 72.6) (end 120.933001 72.6) (width 1.5) (layer "B.Cu") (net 5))
 (segment (start 89.5 113.5) (end 97.3 121.3) (width 1.5) (layer "B.Cu") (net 5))
 (segment (start 120.933001 72.6) (end 118.54 74.993001) (width 1.5) (layer "B.Cu") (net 5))
 (segment (start 118.54 74.993001) (end 118.54 75) (width 1.5) (layer "B.Cu") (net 5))
 (segment (start 149.752792 121.3) (end 150.78 120.272792) (width 1.5) (layer "B.Cu") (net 5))
 (segment (start 91.68 76.202081) (end 97.477919 82) (width 1.5) (layer "B.Cu") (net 5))
 (segment (start 94.073001 72.6) (end 91.68 74.993001) (width 1.5) (layer "B.Cu") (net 5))
 (segment (start 97.477919 82) (end 140.38 82) (width 1.5) (layer "B.Cu") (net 5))
 (segment (start 116.14 72.6) (end 94.073001 72.6) (width 1.5) (layer "B.Cu") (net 5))
 (segment (start 97.3 121.3) (end 149.752792 121.3) (width 1.5) (layer "B.Cu") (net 5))
 (segment (start 91.68 74.993001) (end 91.68 75) (width 1.5) (layer "B.Cu") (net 5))
 (segment (start 141.4 76.202081) (end 139.402081 78.2) (width 1.5) (layer "B.Cu") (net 10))
 (segment (start 153 84) (end 156 87) (width 1.5) (layer "B.Cu") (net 10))
 (segment (start 143.97 77.57) (end 141.4 75) (width 1.5) (layer "B.Cu") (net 10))
 (segment (start 149.647208 84) (end 153 84) (width 1.5) (layer "B.Cu") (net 10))
 (segment (start 151.54 70) (end 143.97 77.57) (width 1.5) (layer "B.Cu") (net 10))
 (segment (start 156 87) (end 156 116.32) (width 1.5) (layer "B.Cu") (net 10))
 (segment (start 147.92 81.52) (end 147.92 87) (width 1.5) (layer "B.Cu") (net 10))
 (segment (start 139.402081 78.2) (end 117.74 78.2) (width 1.5) (layer "B.Cu") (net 10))
 (segment (start 117.74 78.2) (end 114.54 75) (width 1.5) (layer "B.Cu") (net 10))
 (segment (start 147.92 87) (end 147.92 85.727208) (width 1.5) (layer "B.Cu") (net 10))
 (segment (start 156 116.32) (end 153.32 119) (width 1.5) (layer "B.Cu") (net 10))
 (segment (start 141.4 75) (end 141.4 76.202081) (width 1.5) (layer "B.Cu") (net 10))
 (segment (start 147.92 85.727208) (end 149.647208 84) (width 1.5) (layer "B.Cu") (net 10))
 (segment (start 141.4 75) (end 147.92 81.52) (width 1.5) (layer "B.Cu") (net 10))
 (segment (start 109.46 87.7) (end 110.638 86.522) (width 0.254) (layer "F.Cu") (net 51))
 (segment (start 113.178 87.212056) (end 113.178 88.234532) (width 0.254) (layer "F.Cu") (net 51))
 (segment (start 126.608 93.091345) (end 126.608 94.108655) (width 0.254) (layer "F.Cu") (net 51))
 (segment (start 116.915 95.295) (end 115.22 93.6) (width 0.254) (layer "F.Cu") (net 51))
 (segment (start 122.606655 89.09) (end 126.608 93.091345) (width 0.254) (layer "F.Cu") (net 51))
 (segment (start 125.421655 95.295) (end 116.915 95.295) (width 0.254) (layer "F.Cu") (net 51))
 (segment (start 113.178 88.234532) (end 114.033468 89.09) (width 0.254) (layer "F.Cu") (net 51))
 (segment (start 126.608 94.108655) (end 125.421655 95.295) (width 0.254) (layer "F.Cu") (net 51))
 (segment (start 110.638 86.522) (end 112.487944 86.522) (width 0.254) (layer "F.Cu") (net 51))
 (segment (start 112.487944 86.522) (end 113.178 87.212056) (width 0.254) (layer "F.Cu") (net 51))
 (segment (start 114.033468 89.09) (end 122.606655 89.09) (width 0.254) (layer "F.Cu") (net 51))
 (segment (start 117.245 90.545) (end 120.3 93.6) (width 0.254) (layer "F.Cu") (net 53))
 (segment (start 102.145 90.545) (end 117.245 90.545) (width 0.254) (layer "F.Cu") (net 53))
 (segment (start 99.3 87.7) (end 102.145 90.545) (width 0.254) (layer "F.Cu") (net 53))
 (segment (start 121.08 87.7) (end 121.860123 87.7) (width 0.254) (layer "F.Cu") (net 12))
 (segment (start 121.860123 87.7) (end 126.532123 92.372) (width 0.254) (layer "F.Cu") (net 12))
 (segment (start 129.148 110.152) (end 120.3 119) (width 0.254) (layer "F.Cu") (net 12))
 (segment (start 128.428655 92.372) (end 129.148 93.091345) (width 0.254) (layer "F.Cu") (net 12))
 (segment (start 129.148 93.091345) (end 129.148 110.152) (width 0.254) (layer "F.Cu") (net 12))
 (segment (start 126.532123 92.372) (end 128.428655 92.372) (width 0.254) (layer "F.Cu") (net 12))
 (segment (start 146.46 91) (end 130.52 91) (width 0.254) (layer "B.Cu") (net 28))
 (segment (start 150.46 87) (end 146.46 91) (width 0.254) (layer "B.Cu") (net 28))
 (segment (start 130.52 91) (end 127.92 93.6) (width 0.254) (layer "B.Cu") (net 28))
 (segment (start 91.458589 85.612) (end 90.047 87.023589) (width 0.254) (layer "F.Cu") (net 32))
 (segment (start 90.047 87.023589) (end 90.047 101.447) (width 0.254) (layer "F.Cu") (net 32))
 (segment (start 90.047 101.447) (end 107.6 119) (width 0.254) (layer "F.Cu") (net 32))
 (segment (start 104.832 85.612) (end 91.458589 85.612) (width 0.254) (layer "F.Cu") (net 32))
 (segment (start 106.92 87.7) (end 104.832 85.612) (width 0.254) (layer "F.Cu") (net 32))
 (segment (start 95.582 86.522) (end 93.732056 86.522) (width 0.254) (layer "F.Cu") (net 48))
 (segment (start 96.76 87.7) (end 95.582 86.522) (width 0.254) (layer "F.Cu") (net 48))
 (segment (start 93.732056 86.522) (end 93.042 87.212056) (width 0.254) (layer "F.Cu") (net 48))
 (segment (start 96.854056 92) (end 106 92) (width 0.254) (layer "F.Cu") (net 48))
 (segment (start 93.042 87.212056) (end 93.042 88.187944) (width 0.254) (layer "F.Cu") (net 48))
 (segment (start 93.042 88.187944) (end 96.854056 92) (width 0.254) (layer "F.Cu") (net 48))
 (segment (start 106 92) (end 107.6 93.6) (width 0.254) (layer "F.Cu") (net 48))
 (segment (start 97.52 91) (end 110.08 91) (width 0.254) (layer "F.Cu") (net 50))
 (segment (start 94.22 87.7) (end 97.52 91) (width 0.254) (layer "F.Cu") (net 50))
 (segment (start 110.08 91) (end 112.68 93.6) (width 0.254) (layer "F.Cu") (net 50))
 (segment (start 120.808655 120.228) (end 113.908 120.228) (width 0.254) (layer "F.Cu") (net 13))
 (segment (start 121.528 118.491345) (end 121.528 119.508655) (width 0.254) (layer "F.Cu") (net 13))
 (segment (start 123.62 87.7) (end 124.400122 87.7) (width 0.254) (layer "F.Cu") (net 13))
 (segment (start 131.688 108.331345) (end 121.528 118.491345) (width 0.254) (layer "F.Cu") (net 13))
 (segment (start 131.688 93.091345) (end 131.688 108.331345) (width 0.254) (layer "F.Cu") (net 13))
 (segment (start 130.596655 92) (end 131.688 93.091345) (width 0.254) (layer "F.Cu") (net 13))
 (segment (start 121.528 119.508655) (end 120.808655 120.228) (width 0.254) (layer "F.Cu") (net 13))
 (segment (start 128.700122 92) (end 130.596655 92) (width 0.254) (layer "F.Cu") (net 13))
 (segment (start 113.908 120.228) (end 112.68 119) (width 0.254) (layer "F.Cu") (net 13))
 (segment (start 124.400122 87.7) (end 128.700122 92) (width 0.254) (layer "F.Cu") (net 13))
 (segment (start 91.647056 86.067) (end 90.502 87.212056) (width 0.254) (layer "F.Cu") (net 35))
 (segment (start 90.502 87.212056) (end 90.502 91.742) (width 0.254) (layer "F.Cu") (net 35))
 (segment (start 90.502 91.742) (end 117.76 119) (width 0.254) (layer "F.Cu") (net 35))
 (segment (start 104.38 87.7) (end 102.747 86.067) (width 0.254) (layer "F.Cu") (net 35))
 (segment (start 102.747 86.067) (end 91.647056 86.067) (width 0.254) (layer "F.Cu") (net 35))
 (segment (start 128.7 87.7) (end 132.09 91.09) (width 0.254) (layer "F.Cu") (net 15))
 (segment (start 136.768 108.331345) (end 144.388 115.951345) (width 0.254) (layer "F.Cu") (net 15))
 (segment (start 141.848 120.228) (end 140.62 119) (width 0.254) (layer "F.Cu") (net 15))
 (segment (start 136.768 93.091345) (end 136.768 108.331345) (width 0.254) (layer "F.Cu") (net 15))
 (segment (start 144.388 115.951345) (end 144.388 119.508655) (width 0.254) (layer "F.Cu") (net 15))
 (segment (start 144.388 119.508655) (end 143.668655 120.228) (width 0.254) (layer "F.Cu") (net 15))
 (segment (start 132.09 91.09) (end 134.766655 91.09) (width 0.254) (layer "F.Cu") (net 15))
 (segment (start 134.766655 91.09) (end 136.768 93.091345) (width 0.254) (layer "F.Cu") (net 15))
 (segment (start 143.668655 120.228) (end 141.848 120.228) (width 0.254) (layer "F.Cu") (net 15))
 (segment (start 119 94.84) (end 117.76 93.6) (width 0.254) (layer "F.Cu") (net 52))
 (segment (start 113.845 89.545) (end 120.545 89.545) (width 0.254) (layer "F.Cu") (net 52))
 (segment (start 112 87.7) (end 113.845 89.545) (width 0.254) (layer "F.Cu") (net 52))
 (segment (start 124.068 93.068) (end 124.068 94.108655) (width 0.254) (layer "F.Cu") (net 52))
 (segment (start 120.545 89.545) (end 124.068 93.068) (width 0.254) (layer "F.Cu") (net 52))
 (segment (start 124.068 94.108655) (end 123.336655 94.84) (width 0.254) (layer "F.Cu") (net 52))
 (segment (start 123.336655 94.84) (end 119 94.84) (width 0.254) (layer "F.Cu") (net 52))
 (segment (start 94.38 85) (end 111.84 85) (width 0.254) (layer "B.Cu") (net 11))
 (segment (start 138.7 85) (end 141.4 87.7) (width 0.254) (layer "B.Cu") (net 11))
 (segment (start 121 85) (end 138.7 85) (width 0.254) (layer "B.Cu") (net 11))
 (segment (start 118.54 87.7) (end 121 85.24) (width 0.254) (layer "B.Cu") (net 11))
 (segment (start 99.98 96) (end 91.68 87.7) (width 0.254) (layer "B.Cu") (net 11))
 (segment (start 121 85.24) (end 121 85) (width 0.254) (layer "B.Cu") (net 11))
 (segment (start 111.84 85) (end 114.54 87.7) (width 0.254) (layer "B.Cu") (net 11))
 (segment (start 99.98 119) (end 99.98 96) (width 0.254) (layer "B.Cu") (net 11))
 (segment (start 114.54 87.7) (end 118.54 87.7) (width 0.254) (layer "B.Cu") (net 11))
 (segment (start 91.68 87.7) (end 94.38 85) (width 0.254) (layer "B.Cu") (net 11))
 (segment (start 132.06 92) (end 130.46 93.6) (width 0.254) (layer "B.Cu") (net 29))
 (segment (start 148 92) (end 132.06 92) (width 0.254) (layer "B.Cu") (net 29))
 (segment (start 153 87) (end 148 92) (width 0.254) (layer "B.Cu") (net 29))
 (segment (start 119.24 90) (end 122.84 93.6) (width 0.254) (layer "F.Cu") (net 54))
 (segment (start 101.84 87.7) (end 104.14 90) (width 0.254) (layer "F.Cu") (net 54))
 (segment (start 104.14 90) (end 119.24 90) (width 0.254) (layer "F.Cu") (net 54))
 (segment (start 132.681655 91.545) (end 134.228 93.091345) (width 0.254) (layer "F.Cu") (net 14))
 (segment (start 134.228 110.068) (end 143.16 119) (width 0.254) (layer "F.Cu") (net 14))
 (segment (start 134.228 93.091345) (end 134.228 110.068) (width 0.254) (layer "F.Cu") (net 14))
 (segment (start 126.16 87.7) (end 130.005 91.545) (width 0.254) (layer "F.Cu") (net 14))
 (segment (start 130.005 91.545) (end 132.681655 91.545) (width 0.254) (layer "F.Cu") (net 14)))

